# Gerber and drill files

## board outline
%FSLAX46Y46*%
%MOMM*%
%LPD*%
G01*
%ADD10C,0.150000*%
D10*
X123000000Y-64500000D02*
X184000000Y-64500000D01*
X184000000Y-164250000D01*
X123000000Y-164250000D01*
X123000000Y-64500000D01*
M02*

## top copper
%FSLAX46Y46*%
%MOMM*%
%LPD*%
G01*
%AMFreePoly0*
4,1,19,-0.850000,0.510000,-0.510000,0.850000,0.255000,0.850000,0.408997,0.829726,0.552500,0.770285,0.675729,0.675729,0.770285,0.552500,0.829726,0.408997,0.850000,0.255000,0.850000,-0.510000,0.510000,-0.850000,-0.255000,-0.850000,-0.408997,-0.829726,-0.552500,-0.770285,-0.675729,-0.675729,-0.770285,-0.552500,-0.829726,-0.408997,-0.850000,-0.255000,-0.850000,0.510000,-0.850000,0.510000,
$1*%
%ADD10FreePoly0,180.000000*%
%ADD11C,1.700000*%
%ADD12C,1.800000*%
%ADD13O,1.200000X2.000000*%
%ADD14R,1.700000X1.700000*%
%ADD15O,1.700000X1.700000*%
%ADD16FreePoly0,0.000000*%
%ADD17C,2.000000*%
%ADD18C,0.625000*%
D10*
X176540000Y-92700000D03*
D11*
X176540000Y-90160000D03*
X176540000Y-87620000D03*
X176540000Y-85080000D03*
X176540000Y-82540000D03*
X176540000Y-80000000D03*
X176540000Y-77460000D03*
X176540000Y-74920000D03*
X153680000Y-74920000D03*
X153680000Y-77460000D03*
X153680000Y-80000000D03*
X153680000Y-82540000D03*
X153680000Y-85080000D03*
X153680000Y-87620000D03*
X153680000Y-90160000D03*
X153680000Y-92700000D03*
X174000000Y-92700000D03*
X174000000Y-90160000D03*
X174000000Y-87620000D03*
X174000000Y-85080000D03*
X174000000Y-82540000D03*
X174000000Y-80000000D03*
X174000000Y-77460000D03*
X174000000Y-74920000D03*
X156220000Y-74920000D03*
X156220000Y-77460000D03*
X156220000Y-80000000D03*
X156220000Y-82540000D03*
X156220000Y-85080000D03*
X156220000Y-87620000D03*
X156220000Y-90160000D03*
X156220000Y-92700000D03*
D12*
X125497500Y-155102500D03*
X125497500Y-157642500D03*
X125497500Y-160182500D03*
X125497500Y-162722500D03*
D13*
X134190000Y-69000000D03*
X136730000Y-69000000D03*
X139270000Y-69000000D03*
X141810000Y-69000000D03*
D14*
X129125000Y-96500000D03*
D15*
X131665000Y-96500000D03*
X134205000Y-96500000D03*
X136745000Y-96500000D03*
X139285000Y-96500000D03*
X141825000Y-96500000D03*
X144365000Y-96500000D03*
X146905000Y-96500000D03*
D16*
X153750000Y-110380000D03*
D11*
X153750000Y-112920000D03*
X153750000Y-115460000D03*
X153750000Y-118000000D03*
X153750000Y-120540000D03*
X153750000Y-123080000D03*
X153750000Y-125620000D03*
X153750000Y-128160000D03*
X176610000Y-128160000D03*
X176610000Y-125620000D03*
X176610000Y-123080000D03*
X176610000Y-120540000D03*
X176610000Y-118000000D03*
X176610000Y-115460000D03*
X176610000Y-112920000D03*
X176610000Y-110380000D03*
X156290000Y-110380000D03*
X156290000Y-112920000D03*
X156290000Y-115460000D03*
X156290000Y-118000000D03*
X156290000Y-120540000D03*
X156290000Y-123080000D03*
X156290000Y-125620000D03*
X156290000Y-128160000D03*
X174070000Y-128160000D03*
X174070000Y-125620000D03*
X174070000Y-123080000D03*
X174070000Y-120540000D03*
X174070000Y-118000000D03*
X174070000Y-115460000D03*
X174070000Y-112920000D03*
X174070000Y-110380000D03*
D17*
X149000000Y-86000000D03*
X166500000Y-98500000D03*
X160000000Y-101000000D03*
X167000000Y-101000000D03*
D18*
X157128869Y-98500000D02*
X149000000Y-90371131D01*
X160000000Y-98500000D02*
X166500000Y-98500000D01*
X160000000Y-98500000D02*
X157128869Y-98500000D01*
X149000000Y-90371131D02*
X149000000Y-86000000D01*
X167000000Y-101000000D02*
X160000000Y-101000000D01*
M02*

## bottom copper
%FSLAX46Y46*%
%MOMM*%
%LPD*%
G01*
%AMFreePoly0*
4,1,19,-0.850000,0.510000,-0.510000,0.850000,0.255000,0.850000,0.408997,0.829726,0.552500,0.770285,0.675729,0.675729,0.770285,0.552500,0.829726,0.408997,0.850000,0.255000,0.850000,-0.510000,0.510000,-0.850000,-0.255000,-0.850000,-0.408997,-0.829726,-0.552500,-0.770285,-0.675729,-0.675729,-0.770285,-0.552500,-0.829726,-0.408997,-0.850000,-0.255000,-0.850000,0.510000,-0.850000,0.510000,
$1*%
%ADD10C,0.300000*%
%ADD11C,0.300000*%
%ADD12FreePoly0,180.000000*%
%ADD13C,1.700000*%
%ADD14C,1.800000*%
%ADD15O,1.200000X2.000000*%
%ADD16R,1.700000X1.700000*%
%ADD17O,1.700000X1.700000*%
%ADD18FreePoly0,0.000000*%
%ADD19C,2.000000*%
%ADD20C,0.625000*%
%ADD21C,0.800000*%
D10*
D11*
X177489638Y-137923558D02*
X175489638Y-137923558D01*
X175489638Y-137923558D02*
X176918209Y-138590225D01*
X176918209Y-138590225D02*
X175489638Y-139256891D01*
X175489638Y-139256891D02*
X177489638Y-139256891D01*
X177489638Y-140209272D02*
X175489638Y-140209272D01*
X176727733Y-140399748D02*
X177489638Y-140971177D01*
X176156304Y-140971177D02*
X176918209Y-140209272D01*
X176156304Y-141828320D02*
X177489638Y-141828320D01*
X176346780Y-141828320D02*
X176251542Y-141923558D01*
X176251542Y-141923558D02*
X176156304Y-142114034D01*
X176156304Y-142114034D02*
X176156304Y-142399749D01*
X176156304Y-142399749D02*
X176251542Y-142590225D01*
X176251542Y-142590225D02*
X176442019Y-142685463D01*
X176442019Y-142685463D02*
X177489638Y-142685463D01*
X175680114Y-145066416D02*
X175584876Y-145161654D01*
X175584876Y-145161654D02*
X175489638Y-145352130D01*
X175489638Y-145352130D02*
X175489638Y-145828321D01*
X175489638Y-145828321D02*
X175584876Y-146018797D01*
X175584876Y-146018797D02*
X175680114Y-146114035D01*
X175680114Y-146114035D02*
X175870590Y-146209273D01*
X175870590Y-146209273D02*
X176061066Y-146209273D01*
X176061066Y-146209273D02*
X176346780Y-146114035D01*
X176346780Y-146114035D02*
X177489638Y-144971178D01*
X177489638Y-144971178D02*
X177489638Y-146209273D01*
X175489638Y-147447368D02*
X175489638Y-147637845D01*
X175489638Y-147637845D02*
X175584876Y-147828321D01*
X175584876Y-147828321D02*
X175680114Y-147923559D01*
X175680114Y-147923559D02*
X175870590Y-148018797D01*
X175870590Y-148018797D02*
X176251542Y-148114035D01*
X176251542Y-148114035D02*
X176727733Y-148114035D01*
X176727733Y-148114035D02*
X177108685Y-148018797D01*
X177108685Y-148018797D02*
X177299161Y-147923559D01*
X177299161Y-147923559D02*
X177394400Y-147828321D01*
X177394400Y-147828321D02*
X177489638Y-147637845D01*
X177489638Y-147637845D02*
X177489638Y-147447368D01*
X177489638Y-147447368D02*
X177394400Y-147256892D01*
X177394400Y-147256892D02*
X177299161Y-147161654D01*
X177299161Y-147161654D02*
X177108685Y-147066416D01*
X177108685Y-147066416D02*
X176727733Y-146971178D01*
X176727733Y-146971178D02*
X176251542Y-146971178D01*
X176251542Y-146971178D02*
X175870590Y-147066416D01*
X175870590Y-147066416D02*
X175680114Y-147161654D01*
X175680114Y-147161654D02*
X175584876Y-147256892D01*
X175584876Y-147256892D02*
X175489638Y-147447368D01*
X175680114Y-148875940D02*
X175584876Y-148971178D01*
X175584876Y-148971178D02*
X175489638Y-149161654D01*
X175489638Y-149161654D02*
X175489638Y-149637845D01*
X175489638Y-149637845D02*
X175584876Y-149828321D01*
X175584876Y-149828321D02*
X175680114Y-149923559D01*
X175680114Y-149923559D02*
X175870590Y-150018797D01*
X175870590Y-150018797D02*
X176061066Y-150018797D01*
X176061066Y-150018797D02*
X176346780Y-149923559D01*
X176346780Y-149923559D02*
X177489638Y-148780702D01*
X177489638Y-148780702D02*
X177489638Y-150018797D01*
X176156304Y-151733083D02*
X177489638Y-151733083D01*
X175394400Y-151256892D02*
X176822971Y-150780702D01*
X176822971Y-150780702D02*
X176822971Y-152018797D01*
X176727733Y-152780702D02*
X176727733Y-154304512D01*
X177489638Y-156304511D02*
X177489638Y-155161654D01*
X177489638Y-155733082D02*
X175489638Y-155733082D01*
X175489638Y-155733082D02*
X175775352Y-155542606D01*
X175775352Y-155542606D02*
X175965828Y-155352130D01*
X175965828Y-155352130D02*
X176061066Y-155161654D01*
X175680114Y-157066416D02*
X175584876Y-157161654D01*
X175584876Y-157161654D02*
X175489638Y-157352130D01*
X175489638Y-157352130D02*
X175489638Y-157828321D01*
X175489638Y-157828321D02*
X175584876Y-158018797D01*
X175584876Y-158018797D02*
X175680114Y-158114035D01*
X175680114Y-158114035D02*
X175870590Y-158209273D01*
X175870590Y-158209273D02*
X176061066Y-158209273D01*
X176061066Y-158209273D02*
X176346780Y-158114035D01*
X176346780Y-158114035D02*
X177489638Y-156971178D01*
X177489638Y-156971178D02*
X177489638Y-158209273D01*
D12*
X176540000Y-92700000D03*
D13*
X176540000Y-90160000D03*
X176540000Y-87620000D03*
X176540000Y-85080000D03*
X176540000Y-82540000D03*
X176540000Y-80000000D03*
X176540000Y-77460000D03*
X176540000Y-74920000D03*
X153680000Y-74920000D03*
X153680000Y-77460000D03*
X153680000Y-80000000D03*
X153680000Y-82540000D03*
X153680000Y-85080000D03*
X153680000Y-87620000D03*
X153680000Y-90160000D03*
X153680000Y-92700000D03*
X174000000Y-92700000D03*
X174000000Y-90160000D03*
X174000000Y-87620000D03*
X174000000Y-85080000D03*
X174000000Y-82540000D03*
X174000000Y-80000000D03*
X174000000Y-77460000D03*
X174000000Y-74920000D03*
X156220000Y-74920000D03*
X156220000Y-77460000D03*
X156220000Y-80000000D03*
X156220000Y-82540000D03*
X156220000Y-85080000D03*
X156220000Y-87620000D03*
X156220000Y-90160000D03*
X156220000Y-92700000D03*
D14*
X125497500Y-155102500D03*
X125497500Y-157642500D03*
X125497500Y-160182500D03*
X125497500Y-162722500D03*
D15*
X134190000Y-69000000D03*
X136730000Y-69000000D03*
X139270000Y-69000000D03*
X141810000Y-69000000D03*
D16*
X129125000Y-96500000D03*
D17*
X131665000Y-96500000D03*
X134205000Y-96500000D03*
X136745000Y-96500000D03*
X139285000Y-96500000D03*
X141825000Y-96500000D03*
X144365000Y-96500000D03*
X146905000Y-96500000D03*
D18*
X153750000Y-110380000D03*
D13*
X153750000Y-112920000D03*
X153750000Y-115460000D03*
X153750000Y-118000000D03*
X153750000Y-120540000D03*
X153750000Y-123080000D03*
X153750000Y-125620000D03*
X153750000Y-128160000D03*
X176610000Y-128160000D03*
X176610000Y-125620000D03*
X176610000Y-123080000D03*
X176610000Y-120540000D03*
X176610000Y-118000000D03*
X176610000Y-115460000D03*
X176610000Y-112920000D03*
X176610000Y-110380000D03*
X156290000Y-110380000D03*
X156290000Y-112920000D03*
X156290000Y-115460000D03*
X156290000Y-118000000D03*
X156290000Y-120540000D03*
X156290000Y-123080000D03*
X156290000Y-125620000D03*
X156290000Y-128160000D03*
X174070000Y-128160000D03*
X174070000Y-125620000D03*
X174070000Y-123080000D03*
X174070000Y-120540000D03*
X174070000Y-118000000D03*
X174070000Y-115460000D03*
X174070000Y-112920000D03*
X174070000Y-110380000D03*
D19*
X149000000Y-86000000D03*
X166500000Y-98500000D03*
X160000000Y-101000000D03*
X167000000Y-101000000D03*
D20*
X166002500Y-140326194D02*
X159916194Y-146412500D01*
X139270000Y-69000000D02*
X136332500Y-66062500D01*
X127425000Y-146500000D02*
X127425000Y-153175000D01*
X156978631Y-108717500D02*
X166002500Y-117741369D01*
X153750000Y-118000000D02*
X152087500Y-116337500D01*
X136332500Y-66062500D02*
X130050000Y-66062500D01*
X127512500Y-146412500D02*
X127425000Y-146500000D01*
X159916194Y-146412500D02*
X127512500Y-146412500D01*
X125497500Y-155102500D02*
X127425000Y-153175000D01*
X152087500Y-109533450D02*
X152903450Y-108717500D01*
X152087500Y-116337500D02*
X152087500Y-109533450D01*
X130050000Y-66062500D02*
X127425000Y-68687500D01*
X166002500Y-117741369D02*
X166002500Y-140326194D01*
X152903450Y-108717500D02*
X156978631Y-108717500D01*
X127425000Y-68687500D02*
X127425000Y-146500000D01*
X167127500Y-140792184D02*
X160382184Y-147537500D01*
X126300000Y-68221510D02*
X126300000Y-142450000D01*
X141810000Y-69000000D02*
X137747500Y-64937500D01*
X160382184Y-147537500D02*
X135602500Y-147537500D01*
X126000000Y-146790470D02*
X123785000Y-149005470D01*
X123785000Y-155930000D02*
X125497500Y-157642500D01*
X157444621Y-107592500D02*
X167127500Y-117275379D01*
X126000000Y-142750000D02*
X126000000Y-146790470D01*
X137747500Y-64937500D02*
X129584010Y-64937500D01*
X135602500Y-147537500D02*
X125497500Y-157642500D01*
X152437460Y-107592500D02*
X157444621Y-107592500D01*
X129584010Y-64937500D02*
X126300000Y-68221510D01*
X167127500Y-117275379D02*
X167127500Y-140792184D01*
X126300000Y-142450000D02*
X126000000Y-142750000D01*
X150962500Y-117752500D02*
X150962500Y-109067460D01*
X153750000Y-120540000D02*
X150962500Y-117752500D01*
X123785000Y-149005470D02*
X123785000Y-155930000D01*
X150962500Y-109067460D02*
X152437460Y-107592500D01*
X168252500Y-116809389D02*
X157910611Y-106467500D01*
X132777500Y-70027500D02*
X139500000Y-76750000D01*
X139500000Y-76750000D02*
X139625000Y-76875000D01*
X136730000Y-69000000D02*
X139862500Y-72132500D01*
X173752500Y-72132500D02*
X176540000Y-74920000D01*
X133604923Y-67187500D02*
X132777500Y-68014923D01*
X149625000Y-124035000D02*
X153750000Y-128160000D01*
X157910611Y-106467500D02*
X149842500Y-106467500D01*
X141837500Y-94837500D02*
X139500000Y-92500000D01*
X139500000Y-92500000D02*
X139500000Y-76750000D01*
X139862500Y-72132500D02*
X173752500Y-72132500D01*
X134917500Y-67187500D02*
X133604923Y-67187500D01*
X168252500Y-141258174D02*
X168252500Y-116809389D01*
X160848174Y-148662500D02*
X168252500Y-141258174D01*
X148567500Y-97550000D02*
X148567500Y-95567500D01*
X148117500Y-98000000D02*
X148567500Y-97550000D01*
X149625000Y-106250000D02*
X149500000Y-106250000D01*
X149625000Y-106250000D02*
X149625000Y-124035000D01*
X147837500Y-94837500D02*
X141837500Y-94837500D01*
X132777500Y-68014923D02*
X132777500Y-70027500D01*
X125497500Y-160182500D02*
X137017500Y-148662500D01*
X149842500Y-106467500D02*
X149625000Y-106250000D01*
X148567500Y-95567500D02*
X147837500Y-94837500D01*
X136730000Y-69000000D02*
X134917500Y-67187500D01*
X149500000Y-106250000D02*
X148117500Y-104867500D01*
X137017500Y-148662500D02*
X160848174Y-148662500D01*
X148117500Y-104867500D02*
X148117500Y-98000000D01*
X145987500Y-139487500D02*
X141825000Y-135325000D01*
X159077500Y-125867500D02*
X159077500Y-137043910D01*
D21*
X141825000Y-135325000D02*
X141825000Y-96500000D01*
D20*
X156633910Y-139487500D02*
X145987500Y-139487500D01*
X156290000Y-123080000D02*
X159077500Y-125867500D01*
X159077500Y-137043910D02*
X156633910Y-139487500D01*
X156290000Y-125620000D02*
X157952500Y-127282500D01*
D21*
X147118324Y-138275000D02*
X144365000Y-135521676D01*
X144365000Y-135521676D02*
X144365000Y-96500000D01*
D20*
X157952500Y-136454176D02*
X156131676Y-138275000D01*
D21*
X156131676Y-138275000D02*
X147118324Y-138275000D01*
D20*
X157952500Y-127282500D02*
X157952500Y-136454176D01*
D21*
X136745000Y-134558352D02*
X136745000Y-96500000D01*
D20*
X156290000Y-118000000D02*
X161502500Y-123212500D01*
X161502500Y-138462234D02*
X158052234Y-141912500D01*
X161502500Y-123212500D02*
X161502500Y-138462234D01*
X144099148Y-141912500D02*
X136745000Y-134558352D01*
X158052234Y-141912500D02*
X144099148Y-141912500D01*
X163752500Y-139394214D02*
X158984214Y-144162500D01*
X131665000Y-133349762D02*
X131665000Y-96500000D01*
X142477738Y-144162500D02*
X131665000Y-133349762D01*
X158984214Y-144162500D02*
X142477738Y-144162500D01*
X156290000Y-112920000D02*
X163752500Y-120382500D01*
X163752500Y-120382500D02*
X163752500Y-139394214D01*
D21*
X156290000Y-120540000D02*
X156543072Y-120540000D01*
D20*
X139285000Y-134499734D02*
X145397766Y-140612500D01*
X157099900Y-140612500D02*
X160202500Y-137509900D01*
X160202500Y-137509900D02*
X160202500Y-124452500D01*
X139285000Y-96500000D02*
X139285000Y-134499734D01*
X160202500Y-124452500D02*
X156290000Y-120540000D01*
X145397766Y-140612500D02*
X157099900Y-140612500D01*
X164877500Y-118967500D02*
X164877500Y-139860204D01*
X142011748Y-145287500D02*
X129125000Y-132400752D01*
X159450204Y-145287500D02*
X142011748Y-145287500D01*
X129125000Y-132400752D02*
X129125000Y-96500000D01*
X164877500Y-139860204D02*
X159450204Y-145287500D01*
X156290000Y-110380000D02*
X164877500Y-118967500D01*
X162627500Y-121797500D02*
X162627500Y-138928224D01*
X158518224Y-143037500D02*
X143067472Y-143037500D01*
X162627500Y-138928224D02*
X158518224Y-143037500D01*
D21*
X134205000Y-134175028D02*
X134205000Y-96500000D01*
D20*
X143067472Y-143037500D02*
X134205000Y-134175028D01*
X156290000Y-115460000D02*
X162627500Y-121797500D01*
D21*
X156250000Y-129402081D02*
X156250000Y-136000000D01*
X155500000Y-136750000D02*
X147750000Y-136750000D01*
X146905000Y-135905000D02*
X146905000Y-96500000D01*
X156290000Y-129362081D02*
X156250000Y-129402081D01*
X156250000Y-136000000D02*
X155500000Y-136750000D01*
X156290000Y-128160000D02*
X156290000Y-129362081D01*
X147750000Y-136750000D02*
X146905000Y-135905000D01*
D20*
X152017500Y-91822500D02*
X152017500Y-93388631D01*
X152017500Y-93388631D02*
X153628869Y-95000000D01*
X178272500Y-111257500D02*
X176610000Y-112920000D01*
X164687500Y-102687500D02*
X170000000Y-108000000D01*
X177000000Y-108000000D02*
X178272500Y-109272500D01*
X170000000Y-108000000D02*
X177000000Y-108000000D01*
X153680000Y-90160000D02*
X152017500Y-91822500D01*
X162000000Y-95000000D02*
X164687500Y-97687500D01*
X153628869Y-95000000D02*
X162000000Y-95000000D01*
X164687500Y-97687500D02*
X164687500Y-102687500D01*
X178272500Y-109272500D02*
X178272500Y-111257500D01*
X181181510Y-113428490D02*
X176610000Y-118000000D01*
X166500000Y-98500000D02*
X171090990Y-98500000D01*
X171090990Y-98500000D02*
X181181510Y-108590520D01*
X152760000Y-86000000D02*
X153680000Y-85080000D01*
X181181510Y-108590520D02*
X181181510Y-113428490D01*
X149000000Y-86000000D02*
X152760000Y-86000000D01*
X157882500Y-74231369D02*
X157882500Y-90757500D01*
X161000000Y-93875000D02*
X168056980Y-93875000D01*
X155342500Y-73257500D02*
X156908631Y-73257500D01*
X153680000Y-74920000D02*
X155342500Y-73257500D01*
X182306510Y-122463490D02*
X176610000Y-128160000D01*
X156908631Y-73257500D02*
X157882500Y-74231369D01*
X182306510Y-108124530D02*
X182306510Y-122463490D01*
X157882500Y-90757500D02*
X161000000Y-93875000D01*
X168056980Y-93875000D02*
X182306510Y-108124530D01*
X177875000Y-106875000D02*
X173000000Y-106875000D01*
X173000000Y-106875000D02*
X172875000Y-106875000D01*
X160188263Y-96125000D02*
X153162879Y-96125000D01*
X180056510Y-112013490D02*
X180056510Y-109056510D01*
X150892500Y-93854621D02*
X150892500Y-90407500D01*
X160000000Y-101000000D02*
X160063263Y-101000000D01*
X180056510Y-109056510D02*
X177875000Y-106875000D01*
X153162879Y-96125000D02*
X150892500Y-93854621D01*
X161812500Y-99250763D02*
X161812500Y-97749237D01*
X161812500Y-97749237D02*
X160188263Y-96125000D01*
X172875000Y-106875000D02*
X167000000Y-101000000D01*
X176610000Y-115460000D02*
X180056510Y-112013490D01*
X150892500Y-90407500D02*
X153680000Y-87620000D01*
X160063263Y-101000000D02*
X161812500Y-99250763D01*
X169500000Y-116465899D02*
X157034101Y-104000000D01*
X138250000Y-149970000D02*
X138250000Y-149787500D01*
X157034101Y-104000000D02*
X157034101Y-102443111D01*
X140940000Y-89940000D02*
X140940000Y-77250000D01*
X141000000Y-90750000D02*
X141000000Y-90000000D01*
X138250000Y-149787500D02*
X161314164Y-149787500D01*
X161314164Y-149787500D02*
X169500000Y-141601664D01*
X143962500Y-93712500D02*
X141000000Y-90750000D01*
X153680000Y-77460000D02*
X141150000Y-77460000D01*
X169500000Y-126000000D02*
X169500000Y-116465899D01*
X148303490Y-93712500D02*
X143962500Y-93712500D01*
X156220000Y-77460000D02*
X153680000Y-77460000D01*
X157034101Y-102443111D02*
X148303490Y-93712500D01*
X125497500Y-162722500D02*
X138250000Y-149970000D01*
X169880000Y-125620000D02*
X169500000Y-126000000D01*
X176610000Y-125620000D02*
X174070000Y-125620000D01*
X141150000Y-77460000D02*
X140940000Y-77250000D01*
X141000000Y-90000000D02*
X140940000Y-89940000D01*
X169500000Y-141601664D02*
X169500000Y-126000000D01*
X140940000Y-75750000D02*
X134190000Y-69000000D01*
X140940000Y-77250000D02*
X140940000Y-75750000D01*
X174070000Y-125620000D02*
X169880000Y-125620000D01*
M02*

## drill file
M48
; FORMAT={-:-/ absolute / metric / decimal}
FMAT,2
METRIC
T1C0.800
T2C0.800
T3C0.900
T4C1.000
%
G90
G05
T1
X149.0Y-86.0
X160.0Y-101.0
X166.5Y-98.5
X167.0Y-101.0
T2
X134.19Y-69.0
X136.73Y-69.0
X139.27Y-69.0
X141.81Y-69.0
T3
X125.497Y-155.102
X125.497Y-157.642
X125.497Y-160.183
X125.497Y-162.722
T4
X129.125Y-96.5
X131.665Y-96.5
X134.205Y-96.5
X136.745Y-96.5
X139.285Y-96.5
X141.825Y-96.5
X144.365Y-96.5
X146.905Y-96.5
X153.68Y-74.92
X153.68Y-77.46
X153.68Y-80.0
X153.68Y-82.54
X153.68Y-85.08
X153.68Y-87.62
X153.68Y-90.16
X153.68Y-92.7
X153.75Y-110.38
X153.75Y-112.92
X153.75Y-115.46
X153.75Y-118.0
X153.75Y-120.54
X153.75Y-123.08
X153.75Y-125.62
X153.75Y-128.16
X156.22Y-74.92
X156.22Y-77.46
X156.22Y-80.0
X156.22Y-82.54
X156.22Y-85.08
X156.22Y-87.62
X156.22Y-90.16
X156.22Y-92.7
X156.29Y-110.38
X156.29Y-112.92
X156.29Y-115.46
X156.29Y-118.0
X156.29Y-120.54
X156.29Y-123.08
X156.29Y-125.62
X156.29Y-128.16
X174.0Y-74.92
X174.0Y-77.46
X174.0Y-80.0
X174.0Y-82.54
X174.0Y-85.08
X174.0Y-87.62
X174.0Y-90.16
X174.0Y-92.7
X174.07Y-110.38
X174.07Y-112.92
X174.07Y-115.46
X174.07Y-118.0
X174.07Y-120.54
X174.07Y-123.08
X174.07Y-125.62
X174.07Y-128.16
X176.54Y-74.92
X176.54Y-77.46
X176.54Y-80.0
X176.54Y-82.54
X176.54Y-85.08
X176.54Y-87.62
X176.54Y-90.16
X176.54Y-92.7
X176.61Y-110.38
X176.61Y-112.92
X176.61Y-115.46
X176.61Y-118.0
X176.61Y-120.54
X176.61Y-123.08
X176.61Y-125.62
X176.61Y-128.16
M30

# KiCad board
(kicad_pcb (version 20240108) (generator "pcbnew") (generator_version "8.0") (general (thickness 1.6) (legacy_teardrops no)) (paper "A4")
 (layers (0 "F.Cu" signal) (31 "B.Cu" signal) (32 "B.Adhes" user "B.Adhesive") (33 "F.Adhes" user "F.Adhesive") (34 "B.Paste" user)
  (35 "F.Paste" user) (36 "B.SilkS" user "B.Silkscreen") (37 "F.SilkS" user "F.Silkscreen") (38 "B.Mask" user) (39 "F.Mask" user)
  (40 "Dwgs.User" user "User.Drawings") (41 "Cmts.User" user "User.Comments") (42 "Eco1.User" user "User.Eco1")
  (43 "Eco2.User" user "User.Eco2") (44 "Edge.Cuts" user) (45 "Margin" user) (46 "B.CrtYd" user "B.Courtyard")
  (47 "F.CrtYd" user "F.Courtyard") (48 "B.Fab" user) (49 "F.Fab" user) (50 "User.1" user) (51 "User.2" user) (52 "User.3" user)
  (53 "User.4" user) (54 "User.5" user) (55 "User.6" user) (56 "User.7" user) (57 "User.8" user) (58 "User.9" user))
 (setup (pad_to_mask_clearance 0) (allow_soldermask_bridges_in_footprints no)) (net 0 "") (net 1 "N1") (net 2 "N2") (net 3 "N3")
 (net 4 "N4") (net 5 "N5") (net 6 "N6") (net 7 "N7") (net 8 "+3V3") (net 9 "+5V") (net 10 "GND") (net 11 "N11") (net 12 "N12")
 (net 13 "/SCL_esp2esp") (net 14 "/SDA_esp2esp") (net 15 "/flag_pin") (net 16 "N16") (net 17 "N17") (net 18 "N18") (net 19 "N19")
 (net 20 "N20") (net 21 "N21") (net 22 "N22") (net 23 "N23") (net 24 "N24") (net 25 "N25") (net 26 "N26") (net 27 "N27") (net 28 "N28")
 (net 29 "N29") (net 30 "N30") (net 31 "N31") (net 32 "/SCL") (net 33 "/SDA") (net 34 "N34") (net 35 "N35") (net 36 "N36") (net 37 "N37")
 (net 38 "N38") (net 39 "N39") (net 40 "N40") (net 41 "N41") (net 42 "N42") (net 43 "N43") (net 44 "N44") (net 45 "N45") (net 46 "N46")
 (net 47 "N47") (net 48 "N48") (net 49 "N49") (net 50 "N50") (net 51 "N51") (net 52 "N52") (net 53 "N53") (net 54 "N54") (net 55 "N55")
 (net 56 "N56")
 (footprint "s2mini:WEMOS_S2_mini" (layer "F.Cu") (at 176.54 92.7 180)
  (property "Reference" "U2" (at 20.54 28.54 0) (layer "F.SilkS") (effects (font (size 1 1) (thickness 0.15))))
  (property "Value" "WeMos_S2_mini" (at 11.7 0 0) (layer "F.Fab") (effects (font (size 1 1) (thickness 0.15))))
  (pad "1" thru_hole roundrect (at 0 0 180) (size 1.7 1.7) (drill 1) (layers "*.Cu" "*.Mask") (remove_unused_layers no)
   (roundrect_rratio 0.35) (chamfer_ratio 0.2) (chamfer top_left bottom_right) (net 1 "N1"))
  (pad "2" thru_hole circle (at 0 2.54 180) (size 1.7 1.7) (drill 1) (layers "*.Cu" "*.Mask") (remove_unused_layers no) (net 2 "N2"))
  (pad "3" thru_hole circle (at 0 5.08 180) (size 1.7 1.7) (drill 1) (layers "*.Cu" "*.Mask") (remove_unused_layers no) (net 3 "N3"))
  (pad "4" thru_hole circle (at 0 7.62 180) (size 1.7 1.7) (drill 1) (layers "*.Cu" "*.Mask") (remove_unused_layers no) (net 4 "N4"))
  (pad "5" thru_hole circle (at 0 10.16 180) (size 1.7 1.7) (drill 1) (layers "*.Cu" "*.Mask") (remove_unused_layers no) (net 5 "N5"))
  (pad "6" thru_hole circle (at 0 12.7 180) (size 1.7 1.7) (drill 1) (layers "*.Cu" "*.Mask") (remove_unused_layers no) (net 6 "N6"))
  (pad "7" thru_hole circle (at 0 15.24 180) (size 1.7 1.7) (drill 1) (layers "*.Cu" "*.Mask") (remove_unused_layers no) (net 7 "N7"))
  (pad "8" thru_hole circle (at 0 17.78 180) (size 1.7 1.7) (drill 1) (layers "*.Cu" "*.Mask") (remove_unused_layers no) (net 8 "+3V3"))
  (pad "9" thru_hole circle (at 22.86 17.78 180) (size 1.7 1.7) (drill 1) (layers "*.Cu" "*.Mask") (remove_unused_layers no) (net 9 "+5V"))
  (pad "10" thru_hole circle (at 22.86 15.24 180) (size 1.7 1.7) (drill 1) (layers "*.Cu" "*.Mask") (remove_unused_layers no) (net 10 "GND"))
  (pad "11" thru_hole circle (at 22.86 12.7 180) (size 1.7 1.7) (drill 1) (layers "*.Cu" "*.Mask") (remove_unused_layers no) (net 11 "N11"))
  (pad "12" thru_hole circle (at 22.86 10.16 180) (size 1.7 1.7) (drill 1) (layers "*.Cu" "*.Mask") (remove_unused_layers no) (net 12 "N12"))
  (pad "13" thru_hole circle (at 22.86 7.62 180) (size 1.7 1.7) (drill 1) (layers "*.Cu" "*.Mask") (remove_unused_layers no)
   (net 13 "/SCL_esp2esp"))
  (pad "14" thru_hole circle (at 22.86 5.08 180) (size 1.7 1.7) (drill 1) (layers "*.Cu" "*.Mask") (remove_unused_layers no)
   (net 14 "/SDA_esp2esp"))
  (pad "15" thru_hole circle (at 22.86 2.54 180) (size 1.7 1.7) (drill 1) (layers "*.Cu" "*.Mask") (remove_unused_layers no)
   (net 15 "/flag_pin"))
  (pad "16" thru_hole circle (at 22.86 0 180) (size 1.7 1.7) (drill 1) (layers "*.Cu" "*.Mask") (remove_unused_layers no) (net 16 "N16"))
  (pad "17" thru_hole circle (at 2.54 0 180) (size 1.7 1.7) (drill 1) (layers "*.Cu" "*.Mask") (remove_unused_layers no) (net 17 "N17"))
  (pad "18" thru_hole circle (at 2.54 2.54 180) (size 1.7 1.7) (drill 1) (layers "*.Cu" "*.Mask") (remove_unused_layers no) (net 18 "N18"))
  (pad "19" thru_hole circle (at 2.54 5.08 180) (size 1.7 1.7) (drill 1) (layers "*.Cu" "*.Mask") (remove_unused_layers no) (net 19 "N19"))
  (pad "20" thru_hole circle (at 2.54 7.62 180) (size 1.7 1.7) (drill 1) (layers "*.Cu" "*.Mask") (remove_unused_layers no) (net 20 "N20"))
  (pad "21" thru_hole circle (at 2.54 10.16 180) (size 1.7 1.7) (drill 1) (layers "*.Cu" "*.Mask") (remove_unused_layers no) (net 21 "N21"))
  (pad "22" thru_hole circle (at 2.54 12.7 180) (size 1.7 1.7) (drill 1) (layers "*.Cu" "*.Mask") (remove_unused_layers no) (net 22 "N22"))
  (pad "23" thru_hole circle (at 2.54 15.24 180) (size 1.7 1.7) (drill 1) (layers "*.Cu" "*.Mask") (remove_unused_layers no) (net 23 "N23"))
  (pad "24" thru_hole circle (at 2.54 17.78 180) (size 1.7 1.7) (drill 1) (layers "*.Cu" "*.Mask") (remove_unused_layers no) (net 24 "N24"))
  (pad "25" thru_hole circle (at 20.32 17.78 180) (size 1.7 1.7) (drill 1) (layers "*.Cu" "*.Mask") (remove_unused_layers no) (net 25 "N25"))
  (pad "26" thru_hole circle (at 20.32 15.24 180) (size 1.7 1.7) (drill 1) (layers "*.Cu" "*.Mask") (remove_unused_layers no) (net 10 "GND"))
  (pad "27" thru_hole circle (at 20.32 12.7 180) (size 1.7 1.7) (drill 1) (layers "*.Cu" "*.Mask") (remove_unused_layers no) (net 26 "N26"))
  (pad "28" thru_hole circle (at 20.32 10.16 180) (size 1.7 1.7) (drill 1) (layers "*.Cu" "*.Mask") (remove_unused_layers no) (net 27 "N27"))
  (pad "29" thru_hole circle (at 20.32 7.62 180) (size 1.7 1.7) (drill 1) (layers "*.Cu" "*.Mask") (remove_unused_layers no) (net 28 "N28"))
  (pad "30" thru_hole circle (at 20.32 5.08 180) (size 1.7 1.7) (drill 1) (layers "*.Cu" "*.Mask") (remove_unused_layers no) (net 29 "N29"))
  (pad "31" thru_hole circle (at 20.32 2.54 180) (size 1.7 1.7) (drill 1) (layers "*.Cu" "*.Mask") (remove_unused_layers no) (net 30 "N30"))
  (pad "32" thru_hole circle (at 20.32 0 180) (size 1.7 1.7) (drill 1) (layers "*.Cu" "*.Mask") (remove_unused_layers no) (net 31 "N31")))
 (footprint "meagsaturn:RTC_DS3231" (layer "F.Cu") (at 163.5975 170.3425 180)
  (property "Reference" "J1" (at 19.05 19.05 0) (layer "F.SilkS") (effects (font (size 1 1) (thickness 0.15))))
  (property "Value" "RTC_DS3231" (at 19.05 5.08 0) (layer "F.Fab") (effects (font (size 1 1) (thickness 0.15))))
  (pad "1" thru_hole circle (at 38.1 15.24 180) (size 1.8 1.8) (drill 0.9) (layers "*.Cu" "*.Mask") (remove_unused_layers no)
   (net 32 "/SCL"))
  (pad "2" thru_hole circle (at 38.1 12.7 180) (size 1.8 1.8) (drill 0.9) (layers "*.Cu" "*.Mask") (remove_unused_layers no) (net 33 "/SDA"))
  (pad "3" thru_hole circle (at 38.1 10.16 180) (size 1.8 1.8) (drill 0.9) (layers "*.Cu" "*.Mask") (remove_unused_layers no) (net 8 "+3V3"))
  (pad "4" thru_hole circle (at 38.1 7.62 180) (size 1.8 1.8) (drill 0.9) (layers "*.Cu" "*.Mask") (remove_unused_layers no) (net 10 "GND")))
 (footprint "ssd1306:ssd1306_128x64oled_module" (layer "F.Cu") (at 138 69)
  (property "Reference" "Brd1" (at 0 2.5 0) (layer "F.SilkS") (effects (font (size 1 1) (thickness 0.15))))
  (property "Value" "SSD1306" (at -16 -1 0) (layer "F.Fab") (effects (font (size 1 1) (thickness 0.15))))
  (pad "1" thru_hole oval (at -3.81 0) (size 1.2 2) (drill 0.8) (layers "*.Cu" "*.Mask") (remove_unused_layers no) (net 10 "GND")
   (thermal_bridge_angle 45))
  (pad "2" thru_hole oval (at -1.27 0) (size 1.2 2) (drill 0.8) (layers "*.Cu" "*.Mask") (remove_unused_layers no) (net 8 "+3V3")
   (thermal_bridge_angle 45))
  (pad "3" thru_hole oval (at 1.27 0) (size 1.2 2) (drill 0.8) (layers "*.Cu" "*.Mask") (remove_unused_layers no) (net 32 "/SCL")
   (thermal_bridge_angle 45))
  (pad "4" thru_hole oval (at 3.81 0) (size 1.2 2) (drill 0.8) (layers "*.Cu" "*.Mask") (remove_unused_layers no) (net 33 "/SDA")
   (thermal_bridge_angle 45)))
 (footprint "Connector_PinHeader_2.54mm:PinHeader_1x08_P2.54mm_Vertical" (layer "F.Cu") (at 129.125 96.5 90)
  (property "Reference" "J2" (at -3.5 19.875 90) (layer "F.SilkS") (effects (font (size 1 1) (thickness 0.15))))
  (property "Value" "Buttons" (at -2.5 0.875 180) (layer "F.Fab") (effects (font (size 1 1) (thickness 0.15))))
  (pad "1" thru_hole rect (at 0 0 90) (size 1.7 1.7) (drill 1) (layers "*.Cu" "*.Mask") (remove_unused_layers no) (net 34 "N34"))
  (pad "2" thru_hole oval (at 0 2.54 90) (size 1.7 1.7) (drill 1) (layers "*.Cu" "*.Mask") (remove_unused_layers no) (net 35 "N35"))
  (pad "3" thru_hole oval (at 0 5.08 90) (size 1.7 1.7) (drill 1) (layers "*.Cu" "*.Mask") (remove_unused_layers no) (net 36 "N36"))
  (pad "4" thru_hole oval (at 0 7.62 90) (size 1.7 1.7) (drill 1) (layers "*.Cu" "*.Mask") (remove_unused_layers no) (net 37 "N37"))
  (pad "5" thru_hole oval (at 0 10.16 90) (size 1.7 1.7) (drill 1) (layers "*.Cu" "*.Mask") (remove_unused_layers no) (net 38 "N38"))
  (pad "6" thru_hole oval (at 0 12.7 90) (size 1.7 1.7) (drill 1) (layers "*.Cu" "*.Mask") (remove_unused_layers no) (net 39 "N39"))
  (pad "7" thru_hole oval (at 0 15.24 90) (size 1.7 1.7) (drill 1) (layers "*.Cu" "*.Mask") (remove_unused_layers no) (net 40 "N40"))
  (pad "8" thru_hole oval (at 0 17.78 90) (size 1.7 1.7) (drill 1) (layers "*.Cu" "*.Mask") (remove_unused_layers no) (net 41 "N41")))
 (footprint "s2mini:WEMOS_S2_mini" (layer "F.Cu") (at 153.75 110.38)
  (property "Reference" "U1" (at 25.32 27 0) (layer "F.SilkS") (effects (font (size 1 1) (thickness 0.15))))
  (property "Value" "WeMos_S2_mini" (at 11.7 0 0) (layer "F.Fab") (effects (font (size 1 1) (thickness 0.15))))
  (pad "1" thru_hole roundrect (at 0 0) (size 1.7 1.7) (drill 1) (layers "*.Cu" "*.Mask") (remove_unused_layers no) (roundrect_rratio 0.35)
   (chamfer_ratio 0.2) (chamfer top_left bottom_right) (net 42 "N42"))
  (pad "2" thru_hole circle (at 0 2.54) (size 1.7 1.7) (drill 1) (layers "*.Cu" "*.Mask") (remove_unused_layers no) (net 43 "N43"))
  (pad "3" thru_hole circle (at 0 5.08) (size 1.7 1.7) (drill 1) (layers "*.Cu" "*.Mask") (remove_unused_layers no) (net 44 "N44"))
  (pad "4" thru_hole circle (at 0 7.62) (size 1.7 1.7) (drill 1) (layers "*.Cu" "*.Mask") (remove_unused_layers no) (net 32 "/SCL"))
  (pad "5" thru_hole circle (at 0 10.16) (size 1.7 1.7) (drill 1) (layers "*.Cu" "*.Mask") (remove_unused_layers no) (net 33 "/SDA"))
  (pad "6" thru_hole circle (at 0 12.7) (size 1.7 1.7) (drill 1) (layers "*.Cu" "*.Mask") (remove_unused_layers no) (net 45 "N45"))
  (pad "7" thru_hole circle (at 0 15.24) (size 1.7 1.7) (drill 1) (layers "*.Cu" "*.Mask") (remove_unused_layers no) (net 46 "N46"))
  (pad "8" thru_hole circle (at 0 17.78) (size 1.7 1.7) (drill 1) (layers "*.Cu" "*.Mask") (remove_unused_layers no) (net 8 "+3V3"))
  (pad "9" thru_hole circle (at 22.86 17.78) (size 1.7 1.7) (drill 1) (layers "*.Cu" "*.Mask") (remove_unused_layers no) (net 9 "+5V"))
  (pad "10" thru_hole circle (at 22.86 15.24) (size 1.7 1.7) (drill 1) (layers "*.Cu" "*.Mask") (remove_unused_layers no) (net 10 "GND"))
  (pad "11" thru_hole circle (at 22.86 12.7) (size 1.7 1.7) (drill 1) (layers "*.Cu" "*.Mask") (remove_unused_layers no) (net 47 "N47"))
  (pad "12" thru_hole circle (at 22.86 10.16) (size 1.7 1.7) (drill 1) (layers "*.Cu" "*.Mask") (remove_unused_layers no) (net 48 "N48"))
  (pad "13" thru_hole circle (at 22.86 7.62) (size 1.7 1.7) (drill 1) (layers "*.Cu" "*.Mask") (remove_unused_layers no)
   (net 13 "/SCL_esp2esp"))
  (pad "14" thru_hole circle (at 22.86 5.08) (size 1.7 1.7) (drill 1) (layers "*.Cu" "*.Mask") (remove_unused_layers no)
   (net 14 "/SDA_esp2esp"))
  (pad "15" thru_hole circle (at 22.86 2.54) (size 1.7 1.7) (drill 1) (layers "*.Cu" "*.Mask") (remove_unused_layers no)
   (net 15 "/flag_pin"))
  (pad "16" thru_hole circle (at 22.86 0) (size 1.7 1.7) (drill 1) (layers "*.Cu" "*.Mask") (remove_unused_layers no) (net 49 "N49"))
  (pad "17" thru_hole circle (at 2.54 0) (size 1.7 1.7) (drill 1) (layers "*.Cu" "*.Mask") (remove_unused_layers no) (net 34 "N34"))
  (pad "18" thru_hole circle (at 2.54 2.54) (size 1.7 1.7) (drill 1) (layers "*.Cu" "*.Mask") (remove_unused_layers no) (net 35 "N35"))
  (pad "19" thru_hole circle (at 2.54 5.08) (size 1.7 1.7) (drill 1) (layers "*.Cu" "*.Mask") (remove_unused_layers no) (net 36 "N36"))
  (pad "20" thru_hole circle (at 2.54 7.62) (size 1.7 1.7) (drill 1) (layers "*.Cu" "*.Mask") (remove_unused_layers no) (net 37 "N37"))
  (pad "21" thru_hole circle (at 2.54 10.16) (size 1.7 1.7) (drill 1) (layers "*.Cu" "*.Mask") (remove_unused_layers no) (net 38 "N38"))
  (pad "22" thru_hole circle (at 2.54 12.7) (size 1.7 1.7) (drill 1) (layers "*.Cu" "*.Mask") (remove_unused_layers no) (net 39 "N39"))
  (pad "23" thru_hole circle (at 2.54 15.24) (size 1.7 1.7) (drill 1) (layers "*.Cu" "*.Mask") (remove_unused_layers no) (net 40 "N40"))
  (pad "24" thru_hole circle (at 2.54 17.78) (size 1.7 1.7) (drill 1) (layers "*.Cu" "*.Mask") (remove_unused_layers no) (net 41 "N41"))
  (pad "25" thru_hole circle (at 20.32 17.78) (size 1.7 1.7) (drill 1) (layers "*.Cu" "*.Mask") (remove_unused_layers no) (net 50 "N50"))
  (pad "26" thru_hole circle (at 20.32 15.24) (size 1.7 1.7) (drill 1) (layers "*.Cu" "*.Mask") (remove_unused_layers no) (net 10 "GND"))
  (pad "27" thru_hole circle (at 20.32 12.7) (size 1.7 1.7) (drill 1) (layers "*.Cu" "*.Mask") (remove_unused_layers no) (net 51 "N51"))
  (pad "28" thru_hole circle (at 20.32 10.16) (size 1.7 1.7) (drill 1) (layers "*.Cu" "*.Mask") (remove_unused_layers no) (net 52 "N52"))
  (pad "29" thru_hole circle (at 20.32 7.62) (size 1.7 1.7) (drill 1) (layers "*.Cu" "*.Mask") (remove_unused_layers no) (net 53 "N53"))
  (pad "30" thru_hole circle (at 20.32 5.08) (size 1.7 1.7) (drill 1) (layers "*.Cu" "*.Mask") (remove_unused_layers no) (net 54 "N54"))
  (pad "31" thru_hole circle (at 20.32 2.54) (size 1.7 1.7) (drill 1) (layers "*.Cu" "*.Mask") (remove_unused_layers no) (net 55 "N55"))
  (pad "32" thru_hole circle (at 20.32 0) (size 1.7 1.7) (drill 1) (layers "*.Cu" "*.Mask") (remove_unused_layers no) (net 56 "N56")))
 (gr_rect (start 123 64.5) (end 184 164.25) (stroke (width 0.15) (type default)) (fill none) (layer "Edge.Cuts"))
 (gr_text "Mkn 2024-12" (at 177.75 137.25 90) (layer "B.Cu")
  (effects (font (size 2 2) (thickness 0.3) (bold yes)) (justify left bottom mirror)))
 (segment (start 166.0025 140.326194) (end 159.916194 146.4125) (width 0.625) (layer "B.Cu") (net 32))
 (segment (start 139.27 69) (end 136.3325 66.0625) (width 0.625) (layer "B.Cu") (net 32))
 (segment (start 127.425 146.5) (end 127.425 153.175) (width 0.625) (layer "B.Cu") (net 32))
 (segment (start 156.978631 108.7175) (end 166.0025 117.741369) (width 0.625) (layer "B.Cu") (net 32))
 (segment (start 153.75 118) (end 152.0875 116.3375) (width 0.625) (layer "B.Cu") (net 32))
 (segment (start 136.3325 66.0625) (end 130.05 66.0625) (width 0.625) (layer "B.Cu") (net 32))
 (segment (start 127.5125 146.4125) (end 127.425 146.5) (width 0.625) (layer "B.Cu") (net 32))
 (segment (start 159.916194 146.4125) (end 127.5125 146.4125) (width 0.625) (layer "B.Cu") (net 32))
 (segment (start 125.4975 155.1025) (end 127.425 153.175) (width 0.625) (layer "B.Cu") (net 32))
 (segment (start 152.0875 109.53345) (end 152.90345 108.7175) (width 0.625) (layer "B.Cu") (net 32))
 (segment (start 152.0875 116.3375) (end 152.0875 109.53345) (width 0.625) (layer "B.Cu") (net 32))
 (segment (start 130.05 66.0625) (end 127.425 68.6875) (width 0.625) (layer "B.Cu") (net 32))
 (segment (start 166.0025 117.741369) (end 166.0025 140.326194) (width 0.625) (layer "B.Cu") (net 32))
 (segment (start 152.90345 108.7175) (end 156.978631 108.7175) (width 0.625) (layer "B.Cu") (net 32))
 (segment (start 127.425 68.6875) (end 127.425 146.5) (width 0.625) (layer "B.Cu") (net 32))
 (segment (start 167.1275 140.792184) (end 160.382184 147.5375) (width 0.625) (layer "B.Cu") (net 33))
 (segment (start 126.3 68.22151) (end 126.3 142.45) (width 0.625) (layer "B.Cu") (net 33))
 (segment (start 141.81 69) (end 137.7475 64.9375) (width 0.625) (layer "B.Cu") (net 33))
 (segment (start 160.382184 147.5375) (end 135.6025 147.5375) (width 0.625) (layer "B.Cu") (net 33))
 (segment (start 126 146.79047) (end 123.785 149.00547) (width 0.625) (layer "B.Cu") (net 33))
 (segment (start 123.785 155.93) (end 125.4975 157.6425) (width 0.625) (layer "B.Cu") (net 33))
 (segment (start 157.444621 107.5925) (end 167.1275 117.275379) (width 0.625) (layer "B.Cu") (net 33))
 (segment (start 126 142.75) (end 126 146.79047) (width 0.625) (layer "B.Cu") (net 33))
 (segment (start 137.7475 64.9375) (end 129.58401 64.9375) (width 0.625) (layer "B.Cu") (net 33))
 (segment (start 135.6025 147.5375) (end 125.4975 157.6425) (width 0.625) (layer "B.Cu") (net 33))
 (segment (start 152.43746 107.5925) (end 157.444621 107.5925) (width 0.625) (layer "B.Cu") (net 33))
 (segment (start 129.58401 64.9375) (end 126.3 68.22151) (width 0.625) (layer "B.Cu") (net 33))
 (segment (start 167.1275 117.275379) (end 167.1275 140.792184) (width 0.625) (layer "B.Cu") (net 33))
 (segment (start 126.3 142.45) (end 126 142.75) (width 0.625) (layer "B.Cu") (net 33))
 (segment (start 150.9625 117.7525) (end 150.9625 109.06746) (width 0.625) (layer "B.Cu") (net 33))
 (segment (start 153.75 120.54) (end 150.9625 117.7525) (width 0.625) (layer "B.Cu") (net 33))
 (segment (start 123.785 149.00547) (end 123.785 155.93) (width 0.625) (layer "B.Cu") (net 33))
 (segment (start 150.9625 109.06746) (end 152.43746 107.5925) (width 0.625) (layer "B.Cu") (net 33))
 (segment (start 168.2525 116.809389) (end 157.910611 106.4675) (width 0.625) (layer "B.Cu") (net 8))
 (segment (start 132.7775 70.0275) (end 139.5 76.75) (width 0.625) (layer "B.Cu") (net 8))
 (segment (start 139.5 76.75) (end 139.625 76.875) (width 0.625) (layer "B.Cu") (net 8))
 (segment (start 136.73 69) (end 139.8625 72.1325) (width 0.625) (layer "B.Cu") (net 8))
 (segment (start 173.7525 72.1325) (end 176.54 74.92) (width 0.625) (layer "B.Cu") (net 8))
 (segment (start 133.604923 67.1875) (end 132.7775 68.014923) (width 0.625) (layer "B.Cu") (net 8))
 (segment (start 149.625 124.035) (end 153.75 128.16) (width 0.625) (layer "B.Cu") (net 8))
 (segment (start 157.910611 106.4675) (end 149.8425 106.4675) (width 0.625) (layer "B.Cu") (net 8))
 (segment (start 141.8375 94.8375) (end 139.5 92.5) (width 0.625) (layer "B.Cu") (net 8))
 (segment (start 139.5 92.5) (end 139.5 76.75) (width 0.625) (layer "B.Cu") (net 8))
 (segment (start 139.8625 72.1325) (end 173.7525 72.1325) (width 0.625) (layer "B.Cu") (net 8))
 (segment (start 134.9175 67.1875) (end 133.604923 67.1875) (width 0.625) (layer "B.Cu") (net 8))
 (segment (start 168.2525 141.258174) (end 168.2525 116.809389) (width 0.625) (layer "B.Cu") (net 8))
 (segment (start 160.848174 148.6625) (end 168.2525 141.258174) (width 0.625) (layer "B.Cu") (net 8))
 (segment (start 148.5675 97.55) (end 148.5675 95.5675) (width 0.625) (layer "B.Cu") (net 8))
 (segment (start 148.1175 98) (end 148.5675 97.55) (width 0.625) (layer "B.Cu") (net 8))
 (segment (start 149.625 106.25) (end 149.5 106.25) (width 0.625) (layer "B.Cu") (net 8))
 (segment (start 149.625 106.25) (end 149.625 124.035) (width 0.625) (layer "B.Cu") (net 8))
 (segment (start 147.8375 94.8375) (end 141.8375 94.8375) (width 0.625) (layer "B.Cu") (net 8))
 (segment (start 132.7775 68.014923) (end 132.7775 70.0275) (width 0.625) (layer "B.Cu") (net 8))
 (segment (start 125.4975 160.1825) (end 137.0175 148.6625) (width 0.625) (layer "B.Cu") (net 8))
 (segment (start 149.8425 106.4675) (end 149.625 106.25) (width 0.625) (layer "B.Cu") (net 8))
 (segment (start 148.5675 95.5675) (end 147.8375 94.8375) (width 0.625) (layer "B.Cu") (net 8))
 (segment (start 136.73 69) (end 134.9175 67.1875) (width 0.625) (layer "B.Cu") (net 8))
 (segment (start 149.5 106.25) (end 148.1175 104.8675) (width 0.625) (layer "B.Cu") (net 8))
 (segment (start 137.0175 148.6625) (end 160.848174 148.6625) (width 0.625) (layer "B.Cu") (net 8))
 (segment (start 148.1175 104.8675) (end 148.1175 98) (width 0.625) (layer "B.Cu") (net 8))
 (segment (start 145.9875 139.4875) (end 141.825 135.325) (width 0.625) (layer "B.Cu") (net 39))
 (segment (start 159.0775 125.8675) (end 159.0775 137.04391) (width 0.625) (layer "B.Cu") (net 39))
 (segment (start 141.825 135.325) (end 141.825 96.5) (width 0.8) (layer "B.Cu") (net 39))
 (segment (start 156.63391 139.4875) (end 145.9875 139.4875) (width 0.625) (layer "B.Cu") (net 39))
 (segment (start 156.29 123.08) (end 159.0775 125.8675) (width 0.625) (layer "B.Cu") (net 39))
 (segment (start 159.0775 137.04391) (end 156.63391 139.4875) (width 0.625) (layer "B.Cu") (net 39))
 (segment (start 156.29 125.62) (end 157.9525 127.2825) (width 0.625) (layer "B.Cu") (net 40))
 (segment (start 147.118324 138.275) (end 144.365 135.521676) (width 0.8) (layer "B.Cu") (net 40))
 (segment (start 144.365 135.521676) (end 144.365 96.5) (width 0.8) (layer "B.Cu") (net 40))
 (segment (start 157.9525 136.454176) (end 156.131676 138.275) (width 0.625) (layer "B.Cu") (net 40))
 (segment (start 156.131676 138.275) (end 147.118324 138.275) (width 0.8) (layer "B.Cu") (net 40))
 (segment (start 157.9525 127.2825) (end 157.9525 136.454176) (width 0.625) (layer "B.Cu") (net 40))
 (segment (start 136.745 134.558352) (end 136.745 96.5) (width 0.8) (layer "B.Cu") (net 37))
 (segment (start 156.29 118) (end 161.5025 123.2125) (width 0.625) (layer "B.Cu") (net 37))
 (segment (start 161.5025 138.462234) (end 158.052234 141.9125) (width 0.625) (layer "B.Cu") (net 37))
 (segment (start 161.5025 123.2125) (end 161.5025 138.462234) (width 0.625) (layer "B.Cu") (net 37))
 (segment (start 144.099148 141.9125) (end 136.745 134.558352) (width 0.625) (layer "B.Cu") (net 37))
 (segment (start 158.052234 141.9125) (end 144.099148 141.9125) (width 0.625) (layer "B.Cu") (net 37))
 (segment (start 163.7525 139.394214) (end 158.984214 144.1625) (width 0.625) (layer "B.Cu") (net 35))
 (segment (start 131.665 133.349762) (end 131.665 96.5) (width 0.625) (layer "B.Cu") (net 35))
 (segment (start 142.477738 144.1625) (end 131.665 133.349762) (width 0.625) (layer "B.Cu") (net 35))
 (segment (start 158.984214 144.1625) (end 142.477738 144.1625) (width 0.625) (layer "B.Cu") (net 35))
 (segment (start 156.29 112.92) (end 163.7525 120.3825) (width 0.625) (layer "B.Cu") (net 35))
 (segment (start 163.7525 120.3825) (end 163.7525 139.394214) (width 0.625) (layer "B.Cu") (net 35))
 (segment (start 156.29 120.54) (end 156.543072 120.54) (width 0.8) (layer "B.Cu") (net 38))
 (segment (start 139.285 134.499734) (end 145.397766 140.6125) (width 0.625) (layer "B.Cu") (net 38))
 (segment (start 157.0999 140.6125) (end 160.2025 137.5099) (width 0.625) (layer "B.Cu") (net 38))
 (segment (start 160.2025 137.5099) (end 160.2025 124.4525) (width 0.625) (layer "B.Cu") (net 38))
 (segment (start 139.285 96.5) (end 139.285 134.499734) (width 0.625) (layer "B.Cu") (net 38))
 (segment (start 160.2025 124.4525) (end 156.29 120.54) (width 0.625) (layer "B.Cu") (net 38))
 (segment (start 145.397766 140.6125) (end 157.0999 140.6125) (width 0.625) (layer "B.Cu") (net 38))
 (segment (start 164.8775 118.9675) (end 164.8775 139.860204) (width 0.625) (layer "B.Cu") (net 34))
 (segment (start 142.011748 145.2875) (end 129.125 132.400752) (width 0.625) (layer "B.Cu") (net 34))
 (segment (start 159.450204 145.2875) (end 142.011748 145.2875) (width 0.625) (layer "B.Cu") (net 34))
 (segment (start 129.125 132.400752) (end 129.125 96.5) (width 0.625) (layer "B.Cu") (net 34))
 (segment (start 164.8775 139.860204) (end 159.450204 145.2875) (width 0.625) (layer "B.Cu") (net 34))
 (segment (start 156.29 110.38) (end 164.8775 118.9675) (width 0.625) (layer "B.Cu") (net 34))
 (segment (start 162.6275 121.7975) (end 162.6275 138.928224) (width 0.625) (layer "B.Cu") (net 36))
 (segment (start 158.518224 143.0375) (end 143.067472 143.0375) (width 0.625) (layer "B.Cu") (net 36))
 (segment (start 162.6275 138.928224) (end 158.518224 143.0375) (width 0.625) (layer "B.Cu") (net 36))
 (segment (start 134.205 134.175028) (end 134.205 96.5) (width 0.8) (layer "B.Cu") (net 36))
 (segment (start 143.067472 143.0375) (end 134.205 134.175028) (width 0.625) (layer "B.Cu") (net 36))
 (segment (start 156.29 115.46) (end 162.6275 121.7975) (width 0.625) (layer "B.Cu") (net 36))
 (segment (start 156.25 129.402081) (end 156.25 136) (width 0.8) (layer "B.Cu") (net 41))
 (segment (start 155.5 136.75) (end 147.75 136.75) (width 0.8) (layer "B.Cu") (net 41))
 (segment (start 146.905 135.905) (end 146.905 96.5) (width 0.8) (layer "B.Cu") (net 41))
 (segment (start 156.29 129.362081) (end 156.25 129.402081) (width 0.8) (layer "B.Cu") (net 41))
 (segment (start 156.25 136) (end 155.5 136.75) (width 0.8) (layer "B.Cu") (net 41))
 (segment (start 156.29 128.16) (end 156.29 129.362081) (width 0.8) (layer "B.Cu") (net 41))
 (segment (start 147.75 136.75) (end 146.905 135.905) (width 0.8) (layer "B.Cu") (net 41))
 (segment (start 152.0175 91.8225) (end 152.0175 93.388631) (width 0.625) (layer "B.Cu") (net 15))
 (segment (start 152.0175 93.388631) (end 153.628869 95) (width 0.625) (layer "B.Cu") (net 15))
 (segment (start 178.2725 111.2575) (end 176.61 112.92) (width 0.625) (layer "B.Cu") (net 15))
 (segment (start 164.6875 102.6875) (end 170 108) (width 0.625) (layer "B.Cu") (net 15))
 (segment (start 177 108) (end 178.2725 109.2725) (width 0.625) (layer "B.Cu") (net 15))
 (segment (start 170 108) (end 177 108) (width 0.625) (layer "B.Cu") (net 15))
 (segment (start 153.68 90.16) (end 152.0175 91.8225) (width 0.625) (layer "B.Cu") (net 15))
 (segment (start 162 95) (end 164.6875 97.6875) (width 0.625) (layer "B.Cu") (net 15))
 (segment (start 153.628869 95) (end 162 95) (width 0.625) (layer "B.Cu") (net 15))
 (segment (start 164.6875 97.6875) (end 164.6875 102.6875) (width 0.625) (layer "B.Cu") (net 15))
 (segment (start 178.2725 109.2725) (end 178.2725 111.2575) (width 0.625) (layer "B.Cu") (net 15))
 (segment (start 157.128869 98.5) (end 149 90.371131) (width 0.625) (layer "F.Cu") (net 13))
 (segment (start 160 98.5) (end 166.5 98.5) (width 0.625) (layer "F.Cu") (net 13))
 (segment (start 160 98.5) (end 157.128869 98.5) (width 0.625) (layer "F.Cu") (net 13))
 (segment (start 149 90.371131) (end 149 86) (width 0.625) (layer "F.Cu") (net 13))
 (via (at 149 86) (size 2) (drill 0.8) (layers "F.Cu" "B.Cu") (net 13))
 (via (at 166.5 98.5) (size 2) (drill 0.8) (layers "F.Cu" "B.Cu") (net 13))
 (segment (start 181.18151 113.42849) (end 176.61 118) (width 0.625) (layer "B.Cu") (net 13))
 (segment (start 166.5 98.5) (end 171.09099 98.5) (width 0.625) (layer "B.Cu") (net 13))
 (segment (start 171.09099 98.5) (end 181.18151 108.59052) (width 0.625) (layer "B.Cu") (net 13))
 (segment (start 152.76 86) (end 153.68 85.08) (width 0.625) (layer "B.Cu") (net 13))
 (segment (start 181.18151 108.59052) (end 181.18151 113.42849) (width 0.625) (layer "B.Cu") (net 13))
 (segment (start 149 86) (end 152.76 86) (width 0.625) (layer "B.Cu") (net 13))
 (segment (start 157.8825 74.231369) (end 157.8825 90.7575) (width 0.625) (layer "B.Cu") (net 9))
 (segment (start 161 93.875) (end 168.05698 93.875) (width 0.625) (layer "B.Cu") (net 9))
 (segment (start 155.3425 73.2575) (end 156.908631 73.2575) (width 0.625) (layer "B.Cu") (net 9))
 (segment (start 153.68 74.92) (end 155.3425 73.2575) (width 0.625) (layer "B.Cu") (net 9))
 (segment (start 182.30651 122.46349) (end 176.61 128.16) (width 0.625) (layer "B.Cu") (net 9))
 (segment (start 156.908631 73.2575) (end 157.8825 74.231369) (width 0.625) (layer "B.Cu") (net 9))
 (segment (start 182.30651 108.12453) (end 182.30651 122.46349) (width 0.625) (layer "B.Cu") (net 9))
 (segment (start 157.8825 90.7575) (end 161 93.875) (width 0.625) (layer "B.Cu") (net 9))
 (segment (start 168.05698 93.875) (end 182.30651 108.12453) (width 0.625) (layer "B.Cu") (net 9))
 (segment (start 167 101) (end 160 101) (width 0.625) (layer "F.Cu") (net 14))
 (via (at 160 101) (size 2) (drill 0.8) (layers "F.Cu" "B.Cu") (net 14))
 (via (at 167 101) (size 2) (drill 0.8) (layers "F.Cu" "B.Cu") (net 14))
 (segment (start 177.875 106.875) (end 173 106.875) (width 0.625) (layer "B.Cu") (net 14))
 (segment (start 173 106.875) (end 172.875 106.875) (width 0.625) (layer "B.Cu") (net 14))
 (segment (start 160.188263 96.125) (end 153.162879 96.125) (width 0.625) (layer "B.Cu") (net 14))
 (segment (start 180.05651 112.01349) (end 180.05651 109.05651) (width 0.625) (layer "B.Cu") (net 14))
 (segment (start 150.8925 93.854621) (end 150.8925 90.4075) (width 0.625) (layer "B.Cu") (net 14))
 (segment (start 160 101) (end 160.063263 101) (width 0.625) (layer "B.Cu") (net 14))
 (segment (start 180.05651 109.05651) (end 177.875 106.875) (width 0.625) (layer "B.Cu") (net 14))
 (segment (start 153.162879 96.125) (end 150.8925 93.854621) (width 0.625) (layer "B.Cu") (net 14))
 (segment (start 161.8125 99.250763) (end 161.8125 97.749237) (width 0.625) (layer "B.Cu") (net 14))
 (segment (start 161.8125 97.749237) (end 160.188263 96.125) (width 0.625) (layer "B.Cu") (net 14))
 (segment (start 172.875 106.875) (end 167 101) (width 0.625) (layer "B.Cu") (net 14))
 (segment (start 176.61 115.46) (end 180.05651 112.01349) (width 0.625) (layer "B.Cu") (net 14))
 (segment (start 150.8925 90.4075) (end 153.68 87.62) (width 0.625) (layer "B.Cu") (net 14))
 (segment (start 160.063263 101) (end 161.8125 99.250763) (width 0.625) (layer "B.Cu") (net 14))
 (segment (start 169.5 116.465899) (end 157.034101 104) (width 0.625) (layer "B.Cu") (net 10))
 (segment (start 138.25 149.97) (end 138.25 149.7875) (width 0.625) (layer "B.Cu") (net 10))
 (segment (start 157.034101 104) (end 157.034101 102.443111) (width 0.625) (layer "B.Cu") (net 10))
 (segment (start 140.94 89.94) (end 140.94 77.25) (width 0.625) (layer "B.Cu") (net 10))
 (segment (start 141 90.75) (end 141 90) (width 0.625) (layer "B.Cu") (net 10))
 (segment (start 138.25 149.7875) (end 161.314164 149.7875) (width 0.625) (layer "B.Cu") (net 10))
 (segment (start 161.314164 149.7875) (end 169.5 141.601664) (width 0.625) (layer "B.Cu") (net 10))
 (segment (start 143.9625 93.7125) (end 141 90.75) (width 0.625) (layer "B.Cu") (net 10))
 (segment (start 153.68 77.46) (end 141.15 77.46) (width 0.625) (layer "B.Cu") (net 10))
 (segment (start 169.5 126) (end 169.5 116.465899) (width 0.625) (layer "B.Cu") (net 10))
 (segment (start 148.30349 93.7125) (end 143.9625 93.7125) (width 0.625) (layer "B.Cu") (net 10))
 (segment (start 156.22 77.46) (end 153.68 77.46) (width 0.625) (layer "B.Cu") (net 10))
 (segment (start 157.034101 102.443111) (end 148.30349 93.7125) (width 0.625) (layer "B.Cu") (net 10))
 (segment (start 125.4975 162.7225) (end 138.25 149.97) (width 0.625) (layer "B.Cu") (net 10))
 (segment (start 169.88 125.62) (end 169.5 126) (width 0.625) (layer "B.Cu") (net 10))
 (segment (start 176.61 125.62) (end 174.07 125.62) (width 0.625) (layer "B.Cu") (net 10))
 (segment (start 141.15 77.46) (end 140.94 77.25) (width 0.625) (layer "B.Cu") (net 10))
 (segment (start 141 90) (end 140.94 89.94) (width 0.625) (layer "B.Cu") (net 10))
 (segment (start 169.5 141.601664) (end 169.5 126) (width 0.625) (layer "B.Cu") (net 10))
 (segment (start 140.94 75.75) (end 134.19 69) (width 0.625) (layer "B.Cu") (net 10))
 (segment (start 140.94 77.25) (end 140.94 75.75) (width 0.625) (layer "B.Cu") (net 10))
 (segment (start 174.07 125.62) (end 169.88 125.62) (width 0.625) (layer "B.Cu") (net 10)))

